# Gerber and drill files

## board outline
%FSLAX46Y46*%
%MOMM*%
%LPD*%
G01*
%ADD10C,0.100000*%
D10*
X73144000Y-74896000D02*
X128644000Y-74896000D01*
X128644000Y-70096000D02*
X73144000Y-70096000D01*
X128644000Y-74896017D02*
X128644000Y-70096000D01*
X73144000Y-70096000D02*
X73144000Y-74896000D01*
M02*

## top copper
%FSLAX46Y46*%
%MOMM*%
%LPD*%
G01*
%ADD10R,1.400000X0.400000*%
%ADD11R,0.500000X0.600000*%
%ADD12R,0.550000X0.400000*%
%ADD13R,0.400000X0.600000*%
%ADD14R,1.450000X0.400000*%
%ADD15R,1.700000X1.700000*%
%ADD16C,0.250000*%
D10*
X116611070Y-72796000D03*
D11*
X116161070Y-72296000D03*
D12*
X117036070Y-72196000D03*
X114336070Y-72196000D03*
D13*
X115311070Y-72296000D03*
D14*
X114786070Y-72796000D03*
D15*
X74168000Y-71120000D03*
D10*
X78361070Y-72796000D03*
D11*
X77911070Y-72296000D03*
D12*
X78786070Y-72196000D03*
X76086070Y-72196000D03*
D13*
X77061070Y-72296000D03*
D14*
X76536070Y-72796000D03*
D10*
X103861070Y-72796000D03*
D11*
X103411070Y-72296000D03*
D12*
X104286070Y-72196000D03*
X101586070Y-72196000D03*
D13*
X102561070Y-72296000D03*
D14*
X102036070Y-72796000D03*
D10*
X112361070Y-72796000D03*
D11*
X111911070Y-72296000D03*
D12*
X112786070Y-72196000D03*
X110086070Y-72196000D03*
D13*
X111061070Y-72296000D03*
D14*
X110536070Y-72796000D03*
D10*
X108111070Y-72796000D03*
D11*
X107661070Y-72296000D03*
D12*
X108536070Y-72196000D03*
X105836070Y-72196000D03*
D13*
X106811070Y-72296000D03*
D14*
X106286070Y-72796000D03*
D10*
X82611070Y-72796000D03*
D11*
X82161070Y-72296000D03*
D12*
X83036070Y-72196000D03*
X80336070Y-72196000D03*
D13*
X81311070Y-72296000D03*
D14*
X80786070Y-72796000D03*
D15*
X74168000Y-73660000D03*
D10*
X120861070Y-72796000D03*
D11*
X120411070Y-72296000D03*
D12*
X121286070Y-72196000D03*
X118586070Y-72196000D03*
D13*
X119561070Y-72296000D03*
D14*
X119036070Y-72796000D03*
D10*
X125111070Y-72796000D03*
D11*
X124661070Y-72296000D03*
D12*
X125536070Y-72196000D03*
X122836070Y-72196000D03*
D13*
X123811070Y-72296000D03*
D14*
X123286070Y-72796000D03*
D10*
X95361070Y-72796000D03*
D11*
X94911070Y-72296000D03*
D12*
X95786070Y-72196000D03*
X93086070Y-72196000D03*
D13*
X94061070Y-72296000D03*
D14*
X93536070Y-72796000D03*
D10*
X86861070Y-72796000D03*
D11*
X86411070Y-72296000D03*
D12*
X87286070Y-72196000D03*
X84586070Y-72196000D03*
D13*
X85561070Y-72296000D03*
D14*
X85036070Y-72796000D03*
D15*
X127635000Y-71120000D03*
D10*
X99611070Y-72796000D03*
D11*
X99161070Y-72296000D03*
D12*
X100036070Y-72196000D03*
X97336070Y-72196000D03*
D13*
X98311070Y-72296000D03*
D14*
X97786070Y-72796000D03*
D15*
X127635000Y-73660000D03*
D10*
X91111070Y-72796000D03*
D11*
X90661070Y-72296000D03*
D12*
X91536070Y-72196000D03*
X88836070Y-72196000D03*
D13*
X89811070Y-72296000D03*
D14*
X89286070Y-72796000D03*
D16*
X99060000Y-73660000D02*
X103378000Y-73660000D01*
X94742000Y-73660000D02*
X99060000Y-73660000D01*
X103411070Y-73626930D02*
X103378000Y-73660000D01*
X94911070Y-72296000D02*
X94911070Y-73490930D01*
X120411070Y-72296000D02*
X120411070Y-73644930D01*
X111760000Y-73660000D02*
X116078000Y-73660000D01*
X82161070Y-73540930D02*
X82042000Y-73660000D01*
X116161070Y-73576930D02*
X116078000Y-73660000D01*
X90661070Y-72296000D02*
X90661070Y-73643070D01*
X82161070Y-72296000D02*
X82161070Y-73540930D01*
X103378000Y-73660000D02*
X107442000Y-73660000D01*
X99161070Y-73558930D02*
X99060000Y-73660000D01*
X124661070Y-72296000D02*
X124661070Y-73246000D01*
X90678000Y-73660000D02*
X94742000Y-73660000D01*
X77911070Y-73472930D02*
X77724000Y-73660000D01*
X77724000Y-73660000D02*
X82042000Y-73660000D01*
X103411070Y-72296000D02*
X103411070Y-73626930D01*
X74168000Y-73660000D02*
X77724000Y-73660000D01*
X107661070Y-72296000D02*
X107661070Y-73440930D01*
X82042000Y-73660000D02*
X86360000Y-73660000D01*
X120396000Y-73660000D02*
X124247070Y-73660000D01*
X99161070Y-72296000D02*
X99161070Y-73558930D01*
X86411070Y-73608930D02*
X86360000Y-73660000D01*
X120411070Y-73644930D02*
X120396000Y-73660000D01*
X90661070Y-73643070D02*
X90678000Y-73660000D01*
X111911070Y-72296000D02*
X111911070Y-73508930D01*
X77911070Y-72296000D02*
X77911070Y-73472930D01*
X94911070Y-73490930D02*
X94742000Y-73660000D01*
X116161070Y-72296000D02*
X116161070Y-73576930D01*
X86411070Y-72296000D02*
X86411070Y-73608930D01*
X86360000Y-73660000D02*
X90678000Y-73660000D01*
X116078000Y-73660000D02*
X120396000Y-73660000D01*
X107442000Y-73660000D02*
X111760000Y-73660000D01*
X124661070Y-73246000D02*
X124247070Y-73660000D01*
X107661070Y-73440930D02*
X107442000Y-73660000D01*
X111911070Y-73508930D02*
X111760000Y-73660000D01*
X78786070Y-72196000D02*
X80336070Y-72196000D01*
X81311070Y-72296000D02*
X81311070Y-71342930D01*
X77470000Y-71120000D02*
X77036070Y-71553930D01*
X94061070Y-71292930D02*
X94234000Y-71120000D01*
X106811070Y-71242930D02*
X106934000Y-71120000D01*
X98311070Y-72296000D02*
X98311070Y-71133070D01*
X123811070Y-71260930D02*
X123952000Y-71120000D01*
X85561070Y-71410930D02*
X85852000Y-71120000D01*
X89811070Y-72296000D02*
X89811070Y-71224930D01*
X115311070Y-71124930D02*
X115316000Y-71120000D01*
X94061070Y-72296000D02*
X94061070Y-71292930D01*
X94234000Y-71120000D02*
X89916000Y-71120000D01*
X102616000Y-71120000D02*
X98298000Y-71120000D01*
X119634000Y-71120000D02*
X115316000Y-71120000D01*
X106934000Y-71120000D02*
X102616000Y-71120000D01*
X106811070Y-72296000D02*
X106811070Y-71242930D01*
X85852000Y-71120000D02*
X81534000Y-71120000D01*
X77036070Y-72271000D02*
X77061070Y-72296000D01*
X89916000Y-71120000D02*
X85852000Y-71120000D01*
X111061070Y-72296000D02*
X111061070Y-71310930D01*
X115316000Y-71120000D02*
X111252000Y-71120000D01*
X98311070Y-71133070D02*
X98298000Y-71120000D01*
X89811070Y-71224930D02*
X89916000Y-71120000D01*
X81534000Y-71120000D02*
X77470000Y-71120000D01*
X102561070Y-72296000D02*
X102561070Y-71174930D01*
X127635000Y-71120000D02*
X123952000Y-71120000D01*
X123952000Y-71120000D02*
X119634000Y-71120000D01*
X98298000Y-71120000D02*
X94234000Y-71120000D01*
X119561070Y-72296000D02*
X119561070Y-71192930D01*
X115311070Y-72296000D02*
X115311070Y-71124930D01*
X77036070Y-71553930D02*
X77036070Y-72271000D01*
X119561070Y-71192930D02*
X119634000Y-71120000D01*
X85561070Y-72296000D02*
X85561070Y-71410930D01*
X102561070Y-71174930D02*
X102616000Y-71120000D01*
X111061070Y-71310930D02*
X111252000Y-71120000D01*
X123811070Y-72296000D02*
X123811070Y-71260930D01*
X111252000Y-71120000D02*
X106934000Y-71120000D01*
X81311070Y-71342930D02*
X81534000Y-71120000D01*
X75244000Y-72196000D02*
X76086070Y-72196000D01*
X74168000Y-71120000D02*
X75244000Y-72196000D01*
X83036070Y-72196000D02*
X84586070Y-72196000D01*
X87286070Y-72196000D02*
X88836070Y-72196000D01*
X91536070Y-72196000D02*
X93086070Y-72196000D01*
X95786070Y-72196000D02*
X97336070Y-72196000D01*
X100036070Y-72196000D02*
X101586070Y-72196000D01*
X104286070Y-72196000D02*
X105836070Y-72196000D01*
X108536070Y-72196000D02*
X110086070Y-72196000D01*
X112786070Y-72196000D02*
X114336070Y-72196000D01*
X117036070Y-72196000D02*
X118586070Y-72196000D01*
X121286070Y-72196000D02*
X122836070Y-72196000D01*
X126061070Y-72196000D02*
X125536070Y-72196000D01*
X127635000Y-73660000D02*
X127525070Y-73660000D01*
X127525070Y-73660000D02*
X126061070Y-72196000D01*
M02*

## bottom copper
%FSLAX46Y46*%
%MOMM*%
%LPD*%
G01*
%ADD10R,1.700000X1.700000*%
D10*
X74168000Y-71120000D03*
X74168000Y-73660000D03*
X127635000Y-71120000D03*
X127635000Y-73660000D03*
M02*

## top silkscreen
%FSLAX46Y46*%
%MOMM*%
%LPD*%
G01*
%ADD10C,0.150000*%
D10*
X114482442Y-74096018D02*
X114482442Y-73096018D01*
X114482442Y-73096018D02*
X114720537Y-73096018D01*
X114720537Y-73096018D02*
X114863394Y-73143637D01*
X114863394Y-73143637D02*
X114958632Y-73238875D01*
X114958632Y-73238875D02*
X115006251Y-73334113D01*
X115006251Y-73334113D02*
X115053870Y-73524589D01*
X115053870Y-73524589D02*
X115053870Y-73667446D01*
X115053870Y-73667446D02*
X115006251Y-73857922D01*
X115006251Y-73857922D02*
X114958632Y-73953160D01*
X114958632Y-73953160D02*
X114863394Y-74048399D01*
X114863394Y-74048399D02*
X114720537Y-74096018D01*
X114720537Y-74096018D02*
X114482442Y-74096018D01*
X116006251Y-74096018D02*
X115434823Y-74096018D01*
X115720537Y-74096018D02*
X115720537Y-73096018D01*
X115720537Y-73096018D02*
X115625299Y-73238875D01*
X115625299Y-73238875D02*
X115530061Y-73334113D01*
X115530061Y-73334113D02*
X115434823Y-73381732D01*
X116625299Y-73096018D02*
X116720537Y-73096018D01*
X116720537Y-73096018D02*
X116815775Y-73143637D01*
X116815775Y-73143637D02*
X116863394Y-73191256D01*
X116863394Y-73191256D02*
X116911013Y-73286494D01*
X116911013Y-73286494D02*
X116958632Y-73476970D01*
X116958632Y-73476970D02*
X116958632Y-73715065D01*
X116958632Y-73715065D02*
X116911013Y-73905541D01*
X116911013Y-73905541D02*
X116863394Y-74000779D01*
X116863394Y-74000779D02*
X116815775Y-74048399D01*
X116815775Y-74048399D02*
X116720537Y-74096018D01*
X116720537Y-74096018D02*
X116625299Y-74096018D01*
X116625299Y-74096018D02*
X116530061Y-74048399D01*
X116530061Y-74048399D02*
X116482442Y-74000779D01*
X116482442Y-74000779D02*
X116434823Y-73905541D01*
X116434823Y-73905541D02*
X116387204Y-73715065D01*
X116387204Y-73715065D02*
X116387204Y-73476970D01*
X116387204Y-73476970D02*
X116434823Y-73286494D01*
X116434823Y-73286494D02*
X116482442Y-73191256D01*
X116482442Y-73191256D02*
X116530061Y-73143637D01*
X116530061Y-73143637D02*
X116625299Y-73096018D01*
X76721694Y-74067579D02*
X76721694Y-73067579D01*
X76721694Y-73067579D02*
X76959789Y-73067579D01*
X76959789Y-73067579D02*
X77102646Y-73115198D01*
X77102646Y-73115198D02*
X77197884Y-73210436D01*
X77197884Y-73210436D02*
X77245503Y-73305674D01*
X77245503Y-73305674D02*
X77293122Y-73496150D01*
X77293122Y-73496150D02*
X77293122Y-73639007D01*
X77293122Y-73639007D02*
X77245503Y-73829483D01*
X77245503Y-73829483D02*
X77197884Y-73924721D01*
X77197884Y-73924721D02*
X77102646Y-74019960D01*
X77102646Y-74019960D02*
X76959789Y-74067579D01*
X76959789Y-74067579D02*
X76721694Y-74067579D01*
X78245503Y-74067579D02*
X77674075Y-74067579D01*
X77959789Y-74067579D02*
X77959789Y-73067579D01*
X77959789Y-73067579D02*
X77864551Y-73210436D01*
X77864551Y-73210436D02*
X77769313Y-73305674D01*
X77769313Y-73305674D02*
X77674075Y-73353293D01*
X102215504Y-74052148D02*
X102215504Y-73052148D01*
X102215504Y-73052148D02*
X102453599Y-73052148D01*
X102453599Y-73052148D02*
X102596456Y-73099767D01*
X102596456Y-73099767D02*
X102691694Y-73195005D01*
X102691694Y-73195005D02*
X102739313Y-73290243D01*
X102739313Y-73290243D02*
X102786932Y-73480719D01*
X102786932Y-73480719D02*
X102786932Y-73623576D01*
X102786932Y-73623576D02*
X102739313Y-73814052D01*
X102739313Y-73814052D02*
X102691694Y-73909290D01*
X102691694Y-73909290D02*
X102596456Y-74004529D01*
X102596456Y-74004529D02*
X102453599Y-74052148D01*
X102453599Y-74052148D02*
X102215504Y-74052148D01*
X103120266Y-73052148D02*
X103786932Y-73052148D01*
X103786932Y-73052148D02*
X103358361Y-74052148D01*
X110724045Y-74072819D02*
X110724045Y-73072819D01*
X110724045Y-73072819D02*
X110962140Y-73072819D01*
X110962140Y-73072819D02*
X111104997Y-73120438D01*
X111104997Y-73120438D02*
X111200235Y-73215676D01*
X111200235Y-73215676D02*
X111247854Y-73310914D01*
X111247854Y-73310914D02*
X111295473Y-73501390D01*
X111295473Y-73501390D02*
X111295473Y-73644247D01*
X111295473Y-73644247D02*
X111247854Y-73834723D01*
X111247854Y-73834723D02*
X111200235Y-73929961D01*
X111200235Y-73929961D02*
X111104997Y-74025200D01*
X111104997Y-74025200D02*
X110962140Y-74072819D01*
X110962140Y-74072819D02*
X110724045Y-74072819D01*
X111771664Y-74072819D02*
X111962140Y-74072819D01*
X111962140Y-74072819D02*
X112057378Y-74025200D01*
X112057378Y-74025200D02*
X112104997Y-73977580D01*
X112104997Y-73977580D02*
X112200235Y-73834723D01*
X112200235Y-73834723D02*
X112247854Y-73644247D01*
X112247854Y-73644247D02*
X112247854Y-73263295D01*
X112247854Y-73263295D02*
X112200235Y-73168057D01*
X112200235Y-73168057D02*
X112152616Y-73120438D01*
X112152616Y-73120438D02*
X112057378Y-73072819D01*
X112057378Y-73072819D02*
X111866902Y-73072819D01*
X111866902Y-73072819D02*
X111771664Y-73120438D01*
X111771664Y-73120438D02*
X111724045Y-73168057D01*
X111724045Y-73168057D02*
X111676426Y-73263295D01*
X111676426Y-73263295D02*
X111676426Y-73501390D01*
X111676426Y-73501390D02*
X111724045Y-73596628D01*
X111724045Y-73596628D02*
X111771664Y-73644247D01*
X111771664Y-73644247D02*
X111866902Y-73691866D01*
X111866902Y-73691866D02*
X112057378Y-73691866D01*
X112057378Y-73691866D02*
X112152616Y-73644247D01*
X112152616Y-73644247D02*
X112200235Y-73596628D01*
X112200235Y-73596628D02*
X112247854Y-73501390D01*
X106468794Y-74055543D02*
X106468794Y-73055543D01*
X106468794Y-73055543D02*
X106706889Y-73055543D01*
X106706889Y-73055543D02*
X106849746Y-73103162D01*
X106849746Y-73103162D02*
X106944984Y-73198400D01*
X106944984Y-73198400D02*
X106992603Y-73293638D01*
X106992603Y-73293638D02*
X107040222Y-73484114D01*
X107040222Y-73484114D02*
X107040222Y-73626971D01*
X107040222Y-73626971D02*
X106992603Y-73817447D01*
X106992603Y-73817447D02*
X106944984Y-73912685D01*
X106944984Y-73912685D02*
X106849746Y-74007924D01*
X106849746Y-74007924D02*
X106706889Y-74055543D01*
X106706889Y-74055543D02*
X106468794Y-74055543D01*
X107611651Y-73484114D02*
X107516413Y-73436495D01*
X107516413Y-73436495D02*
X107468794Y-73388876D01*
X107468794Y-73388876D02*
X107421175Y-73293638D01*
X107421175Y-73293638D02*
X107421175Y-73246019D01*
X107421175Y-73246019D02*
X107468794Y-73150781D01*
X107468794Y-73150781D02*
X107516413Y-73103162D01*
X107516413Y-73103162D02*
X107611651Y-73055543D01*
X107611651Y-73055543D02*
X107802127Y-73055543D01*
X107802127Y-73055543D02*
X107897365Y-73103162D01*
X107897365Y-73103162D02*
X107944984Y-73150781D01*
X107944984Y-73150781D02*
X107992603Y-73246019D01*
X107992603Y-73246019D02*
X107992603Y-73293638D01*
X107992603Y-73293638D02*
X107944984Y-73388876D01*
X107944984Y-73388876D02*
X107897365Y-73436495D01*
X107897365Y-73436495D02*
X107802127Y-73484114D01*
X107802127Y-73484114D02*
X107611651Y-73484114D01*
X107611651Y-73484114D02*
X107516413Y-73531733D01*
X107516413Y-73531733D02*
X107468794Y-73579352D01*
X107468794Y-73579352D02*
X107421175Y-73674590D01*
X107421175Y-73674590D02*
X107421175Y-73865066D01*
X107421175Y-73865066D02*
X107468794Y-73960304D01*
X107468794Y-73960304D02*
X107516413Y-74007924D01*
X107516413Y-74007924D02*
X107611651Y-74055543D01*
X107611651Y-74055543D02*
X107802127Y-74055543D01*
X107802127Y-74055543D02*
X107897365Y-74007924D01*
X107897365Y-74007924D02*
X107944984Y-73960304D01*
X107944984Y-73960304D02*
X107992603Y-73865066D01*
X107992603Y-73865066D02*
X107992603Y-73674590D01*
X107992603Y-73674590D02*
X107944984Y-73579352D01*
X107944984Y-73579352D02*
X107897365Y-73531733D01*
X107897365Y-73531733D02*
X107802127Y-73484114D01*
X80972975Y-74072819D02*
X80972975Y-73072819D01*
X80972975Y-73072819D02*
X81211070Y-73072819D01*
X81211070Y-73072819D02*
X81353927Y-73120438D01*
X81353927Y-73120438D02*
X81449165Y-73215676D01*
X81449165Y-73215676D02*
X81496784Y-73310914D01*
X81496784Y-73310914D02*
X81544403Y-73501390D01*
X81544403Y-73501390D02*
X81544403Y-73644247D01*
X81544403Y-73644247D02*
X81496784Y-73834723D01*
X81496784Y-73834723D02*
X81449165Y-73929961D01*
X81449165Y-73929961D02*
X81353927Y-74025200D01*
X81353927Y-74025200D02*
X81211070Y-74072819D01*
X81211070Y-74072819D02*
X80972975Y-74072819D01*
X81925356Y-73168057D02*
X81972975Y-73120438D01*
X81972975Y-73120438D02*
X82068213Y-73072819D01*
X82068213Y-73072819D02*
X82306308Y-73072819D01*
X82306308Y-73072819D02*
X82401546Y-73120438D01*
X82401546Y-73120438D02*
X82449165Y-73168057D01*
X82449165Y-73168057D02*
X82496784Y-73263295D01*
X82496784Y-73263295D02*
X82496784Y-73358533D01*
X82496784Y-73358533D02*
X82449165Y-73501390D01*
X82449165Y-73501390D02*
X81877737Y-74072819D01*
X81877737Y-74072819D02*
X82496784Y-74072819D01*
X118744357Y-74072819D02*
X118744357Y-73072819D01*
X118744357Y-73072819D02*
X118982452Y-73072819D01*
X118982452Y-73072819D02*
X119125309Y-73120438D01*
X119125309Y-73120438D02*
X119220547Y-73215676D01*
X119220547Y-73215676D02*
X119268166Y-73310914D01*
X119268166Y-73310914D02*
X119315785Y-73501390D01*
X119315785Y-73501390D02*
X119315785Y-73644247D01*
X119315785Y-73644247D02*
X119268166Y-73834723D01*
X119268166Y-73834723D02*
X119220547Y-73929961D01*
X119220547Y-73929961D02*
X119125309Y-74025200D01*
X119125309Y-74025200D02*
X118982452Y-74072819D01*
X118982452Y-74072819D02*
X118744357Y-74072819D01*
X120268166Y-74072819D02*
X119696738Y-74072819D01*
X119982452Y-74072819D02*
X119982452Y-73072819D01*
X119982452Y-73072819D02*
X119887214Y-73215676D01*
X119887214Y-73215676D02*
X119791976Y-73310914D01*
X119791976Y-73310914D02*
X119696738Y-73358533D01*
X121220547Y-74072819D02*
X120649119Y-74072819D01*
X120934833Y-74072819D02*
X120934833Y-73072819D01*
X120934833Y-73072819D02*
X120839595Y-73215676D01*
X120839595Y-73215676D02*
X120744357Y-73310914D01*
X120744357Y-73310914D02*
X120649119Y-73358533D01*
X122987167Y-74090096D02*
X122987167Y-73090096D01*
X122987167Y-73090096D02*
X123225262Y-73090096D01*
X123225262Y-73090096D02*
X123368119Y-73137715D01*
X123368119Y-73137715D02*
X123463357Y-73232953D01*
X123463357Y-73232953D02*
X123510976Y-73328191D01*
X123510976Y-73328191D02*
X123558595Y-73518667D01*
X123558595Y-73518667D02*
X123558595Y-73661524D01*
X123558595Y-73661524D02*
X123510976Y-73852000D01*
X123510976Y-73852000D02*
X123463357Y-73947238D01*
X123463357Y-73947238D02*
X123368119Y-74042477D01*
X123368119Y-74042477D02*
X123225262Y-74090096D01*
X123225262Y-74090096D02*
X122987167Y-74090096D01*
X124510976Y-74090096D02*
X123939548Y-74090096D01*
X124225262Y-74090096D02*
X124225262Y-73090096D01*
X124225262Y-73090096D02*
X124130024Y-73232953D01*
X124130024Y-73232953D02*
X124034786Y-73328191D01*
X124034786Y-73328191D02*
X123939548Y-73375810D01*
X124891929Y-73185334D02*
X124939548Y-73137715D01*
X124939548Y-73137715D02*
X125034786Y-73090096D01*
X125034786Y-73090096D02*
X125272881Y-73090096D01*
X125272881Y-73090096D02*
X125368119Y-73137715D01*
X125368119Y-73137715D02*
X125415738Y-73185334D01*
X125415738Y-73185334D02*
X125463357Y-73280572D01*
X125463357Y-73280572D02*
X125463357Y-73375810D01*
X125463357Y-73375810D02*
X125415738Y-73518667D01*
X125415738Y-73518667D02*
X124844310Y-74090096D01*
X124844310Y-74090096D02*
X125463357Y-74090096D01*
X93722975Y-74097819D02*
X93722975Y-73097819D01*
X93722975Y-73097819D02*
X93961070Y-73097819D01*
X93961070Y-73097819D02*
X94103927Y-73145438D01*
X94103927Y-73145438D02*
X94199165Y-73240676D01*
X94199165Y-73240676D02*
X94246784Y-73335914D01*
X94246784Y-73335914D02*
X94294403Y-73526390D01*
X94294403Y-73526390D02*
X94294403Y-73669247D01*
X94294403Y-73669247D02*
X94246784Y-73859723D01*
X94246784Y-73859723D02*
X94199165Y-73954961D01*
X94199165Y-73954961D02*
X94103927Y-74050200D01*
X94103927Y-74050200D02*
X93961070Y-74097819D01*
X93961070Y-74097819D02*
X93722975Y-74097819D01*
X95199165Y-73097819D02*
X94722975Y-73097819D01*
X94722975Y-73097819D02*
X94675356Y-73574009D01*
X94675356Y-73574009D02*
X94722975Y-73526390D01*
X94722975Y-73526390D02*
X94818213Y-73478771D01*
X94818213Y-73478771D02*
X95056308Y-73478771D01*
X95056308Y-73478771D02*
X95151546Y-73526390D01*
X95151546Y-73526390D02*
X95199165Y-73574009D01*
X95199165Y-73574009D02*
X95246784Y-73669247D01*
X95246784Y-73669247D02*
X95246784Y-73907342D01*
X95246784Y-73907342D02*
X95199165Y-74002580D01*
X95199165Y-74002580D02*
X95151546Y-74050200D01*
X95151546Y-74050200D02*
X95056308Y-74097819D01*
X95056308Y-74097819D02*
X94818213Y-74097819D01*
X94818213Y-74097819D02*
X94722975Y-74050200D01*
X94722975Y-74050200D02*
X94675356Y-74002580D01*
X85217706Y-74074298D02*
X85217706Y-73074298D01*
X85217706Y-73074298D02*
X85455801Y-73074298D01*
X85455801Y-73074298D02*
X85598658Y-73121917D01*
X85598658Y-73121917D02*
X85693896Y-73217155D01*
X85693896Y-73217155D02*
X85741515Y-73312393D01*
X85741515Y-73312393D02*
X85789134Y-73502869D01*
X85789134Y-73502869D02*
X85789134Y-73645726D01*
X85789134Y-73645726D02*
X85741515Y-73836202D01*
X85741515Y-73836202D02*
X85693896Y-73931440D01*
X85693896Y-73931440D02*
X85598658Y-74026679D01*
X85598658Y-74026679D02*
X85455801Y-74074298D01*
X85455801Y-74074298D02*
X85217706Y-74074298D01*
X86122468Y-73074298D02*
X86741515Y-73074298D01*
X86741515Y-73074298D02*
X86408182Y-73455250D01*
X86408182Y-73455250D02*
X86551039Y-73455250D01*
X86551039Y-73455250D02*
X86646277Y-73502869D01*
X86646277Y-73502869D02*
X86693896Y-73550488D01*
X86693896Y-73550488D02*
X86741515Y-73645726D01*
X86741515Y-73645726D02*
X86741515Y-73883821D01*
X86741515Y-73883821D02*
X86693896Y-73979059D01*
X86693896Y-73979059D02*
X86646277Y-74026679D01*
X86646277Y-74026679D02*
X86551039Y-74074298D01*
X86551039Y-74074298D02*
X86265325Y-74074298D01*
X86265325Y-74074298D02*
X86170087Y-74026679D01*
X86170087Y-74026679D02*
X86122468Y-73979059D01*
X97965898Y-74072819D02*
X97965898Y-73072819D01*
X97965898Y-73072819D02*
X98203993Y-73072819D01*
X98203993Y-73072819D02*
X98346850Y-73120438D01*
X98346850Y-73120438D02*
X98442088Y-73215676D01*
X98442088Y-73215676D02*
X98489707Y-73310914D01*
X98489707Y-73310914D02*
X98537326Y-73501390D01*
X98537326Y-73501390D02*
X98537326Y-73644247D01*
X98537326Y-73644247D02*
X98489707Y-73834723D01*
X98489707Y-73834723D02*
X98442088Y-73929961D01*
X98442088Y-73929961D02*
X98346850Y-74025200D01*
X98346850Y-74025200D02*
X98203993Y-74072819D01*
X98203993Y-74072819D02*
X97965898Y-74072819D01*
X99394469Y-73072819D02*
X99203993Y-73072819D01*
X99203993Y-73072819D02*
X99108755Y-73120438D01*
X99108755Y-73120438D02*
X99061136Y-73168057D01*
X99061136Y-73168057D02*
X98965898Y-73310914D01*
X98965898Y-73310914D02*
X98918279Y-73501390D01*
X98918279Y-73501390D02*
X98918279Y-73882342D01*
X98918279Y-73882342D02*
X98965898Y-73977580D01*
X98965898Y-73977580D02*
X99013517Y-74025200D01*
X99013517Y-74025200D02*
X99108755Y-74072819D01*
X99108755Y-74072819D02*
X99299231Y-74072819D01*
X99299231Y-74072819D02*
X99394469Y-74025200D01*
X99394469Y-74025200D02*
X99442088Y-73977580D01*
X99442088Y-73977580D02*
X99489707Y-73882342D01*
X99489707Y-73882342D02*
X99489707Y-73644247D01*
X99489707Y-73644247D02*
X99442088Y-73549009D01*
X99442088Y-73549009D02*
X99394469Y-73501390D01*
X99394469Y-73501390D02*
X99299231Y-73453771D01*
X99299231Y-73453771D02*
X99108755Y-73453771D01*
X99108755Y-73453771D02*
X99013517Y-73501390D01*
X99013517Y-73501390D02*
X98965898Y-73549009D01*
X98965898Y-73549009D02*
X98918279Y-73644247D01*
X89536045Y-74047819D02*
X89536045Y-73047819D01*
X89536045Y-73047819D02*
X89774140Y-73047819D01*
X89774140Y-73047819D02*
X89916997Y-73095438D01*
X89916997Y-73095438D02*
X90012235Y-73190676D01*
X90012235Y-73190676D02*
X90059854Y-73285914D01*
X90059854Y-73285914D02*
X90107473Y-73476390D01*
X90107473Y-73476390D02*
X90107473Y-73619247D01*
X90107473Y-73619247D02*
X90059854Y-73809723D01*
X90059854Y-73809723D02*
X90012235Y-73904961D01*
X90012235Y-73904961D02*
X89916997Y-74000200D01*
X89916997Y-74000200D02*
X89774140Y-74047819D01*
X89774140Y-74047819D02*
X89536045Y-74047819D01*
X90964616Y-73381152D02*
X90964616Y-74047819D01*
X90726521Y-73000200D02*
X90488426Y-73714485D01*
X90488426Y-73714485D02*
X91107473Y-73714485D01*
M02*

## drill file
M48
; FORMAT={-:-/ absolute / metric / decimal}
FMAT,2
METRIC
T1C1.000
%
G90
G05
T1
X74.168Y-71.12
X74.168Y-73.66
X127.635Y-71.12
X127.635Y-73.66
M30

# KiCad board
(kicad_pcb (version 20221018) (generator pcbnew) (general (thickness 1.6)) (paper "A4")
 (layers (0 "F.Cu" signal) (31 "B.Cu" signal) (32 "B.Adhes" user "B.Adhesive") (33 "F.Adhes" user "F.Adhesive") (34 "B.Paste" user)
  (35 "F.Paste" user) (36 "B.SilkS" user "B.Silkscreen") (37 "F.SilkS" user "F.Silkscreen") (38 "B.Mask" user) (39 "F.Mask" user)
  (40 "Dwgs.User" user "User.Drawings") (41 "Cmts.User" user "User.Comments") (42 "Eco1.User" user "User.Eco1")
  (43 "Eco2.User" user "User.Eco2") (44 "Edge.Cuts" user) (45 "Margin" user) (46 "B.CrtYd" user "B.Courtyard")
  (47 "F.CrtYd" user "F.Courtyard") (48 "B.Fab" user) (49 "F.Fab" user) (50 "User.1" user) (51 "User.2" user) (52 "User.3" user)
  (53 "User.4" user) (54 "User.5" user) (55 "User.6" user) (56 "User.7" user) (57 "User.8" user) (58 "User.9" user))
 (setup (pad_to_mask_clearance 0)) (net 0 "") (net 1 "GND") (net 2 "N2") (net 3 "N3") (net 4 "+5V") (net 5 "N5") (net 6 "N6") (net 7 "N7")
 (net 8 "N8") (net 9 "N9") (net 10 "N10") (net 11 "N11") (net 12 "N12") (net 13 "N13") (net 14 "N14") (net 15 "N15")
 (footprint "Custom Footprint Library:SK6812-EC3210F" (layer "F.Cu") (at 115.71107 72.496 180)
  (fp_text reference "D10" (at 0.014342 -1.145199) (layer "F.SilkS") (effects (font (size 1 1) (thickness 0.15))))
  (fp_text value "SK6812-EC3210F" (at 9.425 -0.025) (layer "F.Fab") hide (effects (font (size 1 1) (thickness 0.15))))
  (pad "1" smd rect (at -0.9 -0.3) (size 1.4 0.4) (layers "F.Cu" "F.Paste" "F.Mask") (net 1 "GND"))
  (pad "1" smd rect (at -0.45 0.2) (size 0.5 0.6) (layers "F.Cu" "F.Paste" "F.Mask") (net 1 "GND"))
  (pad "2" smd rect (at -1.325 0.3) (size 0.55 0.4) (layers "F.Cu" "F.Paste" "F.Mask") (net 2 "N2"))
  (pad "3" smd rect (at 1.375 0.3) (size 0.55 0.4) (layers "F.Cu" "F.Paste" "F.Mask") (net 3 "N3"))
  (pad "4" smd rect (at 0.4 0.2) (size 0.4 0.6) (layers "F.Cu" "F.Paste" "F.Mask") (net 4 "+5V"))
  (pad "4" smd rect (at 0.925 -0.3) (size 1.45 0.4) (layers "F.Cu" "F.Paste" "F.Mask") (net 4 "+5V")))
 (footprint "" (layer "F.Cu") (at 74.168 71.12)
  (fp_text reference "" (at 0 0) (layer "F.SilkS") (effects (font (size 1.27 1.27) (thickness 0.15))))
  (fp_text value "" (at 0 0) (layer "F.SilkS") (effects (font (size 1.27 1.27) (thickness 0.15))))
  (pad "1" thru_hole rect (at 0 0) (size 1.7 1.7) (drill 1) (layers "*.Cu" "*.Mask") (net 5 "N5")))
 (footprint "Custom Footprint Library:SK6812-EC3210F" (layer "F.Cu") (at 77.46107 72.496 180)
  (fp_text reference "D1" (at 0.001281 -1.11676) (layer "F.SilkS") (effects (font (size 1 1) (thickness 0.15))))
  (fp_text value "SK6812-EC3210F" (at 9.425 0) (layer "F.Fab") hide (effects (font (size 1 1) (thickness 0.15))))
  (pad "1" smd rect (at -0.9 -0.3) (size 1.4 0.4) (layers "F.Cu" "F.Paste" "F.Mask") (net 1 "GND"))
  (pad "1" smd rect (at -0.45 0.2) (size 0.5 0.6) (layers "F.Cu" "F.Paste" "F.Mask") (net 1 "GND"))
  (pad "2" smd rect (at -1.325 0.3) (size 0.55 0.4) (layers "F.Cu" "F.Paste" "F.Mask") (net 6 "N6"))
  (pad "3" smd rect (at 1.375 0.3) (size 0.55 0.4) (layers "F.Cu" "F.Paste" "F.Mask") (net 5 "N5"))
  (pad "4" smd rect (at 0.4 0.2) (size 0.4 0.6) (layers "F.Cu" "F.Paste" "F.Mask") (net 4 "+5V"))
  (pad "4" smd rect (at 0.925 -0.3) (size 1.45 0.4) (layers "F.Cu" "F.Paste" "F.Mask") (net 4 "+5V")))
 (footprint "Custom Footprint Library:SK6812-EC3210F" (layer "F.Cu") (at 102.96107 72.496 180)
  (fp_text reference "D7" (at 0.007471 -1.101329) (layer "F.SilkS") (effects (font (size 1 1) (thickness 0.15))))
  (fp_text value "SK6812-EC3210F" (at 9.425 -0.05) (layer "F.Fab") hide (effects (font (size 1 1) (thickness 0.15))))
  (pad "1" smd rect (at -0.9 -0.3) (size 1.4 0.4) (layers "F.Cu" "F.Paste" "F.Mask") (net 1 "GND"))
  (pad "1" smd rect (at -0.45 0.2) (size 0.5 0.6) (layers "F.Cu" "F.Paste" "F.Mask") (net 1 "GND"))
  (pad "2" smd rect (at -1.325 0.3) (size 0.55 0.4) (layers "F.Cu" "F.Paste" "F.Mask") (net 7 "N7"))
  (pad "3" smd rect (at 1.375 0.3) (size 0.55 0.4) (layers "F.Cu" "F.Paste" "F.Mask") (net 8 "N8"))
  (pad "4" smd rect (at 0.4 0.2) (size 0.4 0.6) (layers "F.Cu" "F.Paste" "F.Mask") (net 4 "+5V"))
  (pad "4" smd rect (at 0.925 -0.3) (size 1.45 0.4) (layers "F.Cu" "F.Paste" "F.Mask") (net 4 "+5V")))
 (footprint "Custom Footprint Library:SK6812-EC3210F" (layer "F.Cu") (at 111.46107 72.496 180)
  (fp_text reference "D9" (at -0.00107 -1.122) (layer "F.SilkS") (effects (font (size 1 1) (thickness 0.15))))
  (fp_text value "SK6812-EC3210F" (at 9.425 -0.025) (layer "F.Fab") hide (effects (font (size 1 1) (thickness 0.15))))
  (pad "1" smd rect (at -0.9 -0.3) (size 1.4 0.4) (layers "F.Cu" "F.Paste" "F.Mask") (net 1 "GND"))
  (pad "1" smd rect (at -0.45 0.2) (size 0.5 0.6) (layers "F.Cu" "F.Paste" "F.Mask") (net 1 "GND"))
  (pad "2" smd rect (at -1.325 0.3) (size 0.55 0.4) (layers "F.Cu" "F.Paste" "F.Mask") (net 3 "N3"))
  (pad "3" smd rect (at 1.375 0.3) (size 0.55 0.4) (layers "F.Cu" "F.Paste" "F.Mask") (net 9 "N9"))
  (pad "4" smd rect (at 0.4 0.2) (size 0.4 0.6) (layers "F.Cu" "F.Paste" "F.Mask") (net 4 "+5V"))
  (pad "4" smd rect (at 0.925 -0.3) (size 1.45 0.4) (layers "F.Cu" "F.Paste" "F.Mask") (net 4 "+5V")))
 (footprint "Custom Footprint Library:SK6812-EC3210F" (layer "F.Cu") (at 107.21107 72.496 180)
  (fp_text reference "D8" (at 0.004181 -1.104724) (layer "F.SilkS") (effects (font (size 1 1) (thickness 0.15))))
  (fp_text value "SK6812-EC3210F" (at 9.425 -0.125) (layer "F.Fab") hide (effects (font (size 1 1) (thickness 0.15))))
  (pad "1" smd rect (at -0.9 -0.3) (size 1.4 0.4) (layers "F.Cu" "F.Paste" "F.Mask") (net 1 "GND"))
  (pad "1" smd rect (at -0.45 0.2) (size 0.5 0.6) (layers "F.Cu" "F.Paste" "F.Mask") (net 1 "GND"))
  (pad "2" smd rect (at -1.325 0.3) (size 0.55 0.4) (layers "F.Cu" "F.Paste" "F.Mask") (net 9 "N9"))
  (pad "3" smd rect (at 1.375 0.3) (size 0.55 0.4) (layers "F.Cu" "F.Paste" "F.Mask") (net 7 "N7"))
  (pad "4" smd rect (at 0.4 0.2) (size 0.4 0.6) (layers "F.Cu" "F.Paste" "F.Mask") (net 4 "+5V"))
  (pad "4" smd rect (at 0.925 -0.3) (size 1.45 0.4) (layers "F.Cu" "F.Paste" "F.Mask") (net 4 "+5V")))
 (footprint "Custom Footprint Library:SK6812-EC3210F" (layer "F.Cu") (at 81.71107 72.496 180)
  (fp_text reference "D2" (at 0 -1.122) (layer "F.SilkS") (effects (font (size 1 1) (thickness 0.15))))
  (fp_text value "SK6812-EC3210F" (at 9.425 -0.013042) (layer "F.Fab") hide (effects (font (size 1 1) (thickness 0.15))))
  (pad "1" smd rect (at -0.9 -0.3) (size 1.4 0.4) (layers "F.Cu" "F.Paste" "F.Mask") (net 1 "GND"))
  (pad "1" smd rect (at -0.45 0.2) (size 0.5 0.6) (layers "F.Cu" "F.Paste" "F.Mask") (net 1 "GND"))
  (pad "2" smd rect (at -1.325 0.3) (size 0.55 0.4) (layers "F.Cu" "F.Paste" "F.Mask") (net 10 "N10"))
  (pad "3" smd rect (at 1.375 0.3) (size 0.55 0.4) (layers "F.Cu" "F.Paste" "F.Mask") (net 6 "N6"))
  (pad "4" smd rect (at 0.4 0.2) (size 0.4 0.6) (layers "F.Cu" "F.Paste" "F.Mask") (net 4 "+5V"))
  (pad "4" smd rect (at 0.925 -0.3) (size 1.45 0.4) (layers "F.Cu" "F.Paste" "F.Mask") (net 4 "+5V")))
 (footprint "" (layer "F.Cu") (at 74.168 73.66)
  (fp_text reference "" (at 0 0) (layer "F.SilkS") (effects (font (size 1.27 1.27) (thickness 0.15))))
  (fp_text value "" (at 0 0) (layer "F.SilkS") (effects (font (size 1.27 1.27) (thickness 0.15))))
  (pad "1" thru_hole rect (at 0 0) (size 1.7 1.7) (drill 1) (layers "*.Cu" "*.Mask") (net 1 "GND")))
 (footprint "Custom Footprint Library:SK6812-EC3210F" (layer "F.Cu") (at 119.96107 72.496 180)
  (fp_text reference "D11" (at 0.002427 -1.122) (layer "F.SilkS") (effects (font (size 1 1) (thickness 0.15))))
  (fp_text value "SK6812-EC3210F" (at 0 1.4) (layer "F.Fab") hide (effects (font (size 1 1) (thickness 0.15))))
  (pad "1" smd rect (at -0.9 -0.3) (size 1.4 0.4) (layers "F.Cu" "F.Paste" "F.Mask") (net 1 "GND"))
  (pad "1" smd rect (at -0.45 0.2) (size 0.5 0.6) (layers "F.Cu" "F.Paste" "F.Mask") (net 1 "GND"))
  (pad "2" smd rect (at -1.325 0.3) (size 0.55 0.4) (layers "F.Cu" "F.Paste" "F.Mask") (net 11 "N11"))
  (pad "3" smd rect (at 1.375 0.3) (size 0.55 0.4) (layers "F.Cu" "F.Paste" "F.Mask") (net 2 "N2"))
  (pad "4" smd rect (at 0.4 0.2) (size 0.4 0.6) (layers "F.Cu" "F.Paste" "F.Mask") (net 4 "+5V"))
  (pad "4" smd rect (at 0.925 -0.3) (size 1.45 0.4) (layers "F.Cu" "F.Paste" "F.Mask") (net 4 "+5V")))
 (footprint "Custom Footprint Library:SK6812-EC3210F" (layer "F.Cu") (at 124.21107 72.496 180)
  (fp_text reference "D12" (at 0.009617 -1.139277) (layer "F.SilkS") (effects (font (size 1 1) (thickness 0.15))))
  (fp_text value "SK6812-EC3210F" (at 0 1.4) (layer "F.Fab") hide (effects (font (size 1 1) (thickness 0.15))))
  (pad "1" smd rect (at -0.9 -0.3) (size 1.4 0.4) (layers "F.Cu" "F.Paste" "F.Mask") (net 1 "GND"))
  (pad "1" smd rect (at -0.45 0.2) (size 0.5 0.6) (layers "F.Cu" "F.Paste" "F.Mask") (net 1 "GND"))
  (pad "2" smd rect (at -1.325 0.3) (size 0.55 0.4) (layers "F.Cu" "F.Paste" "F.Mask") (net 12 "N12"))
  (pad "3" smd rect (at 1.375 0.3) (size 0.55 0.4) (layers "F.Cu" "F.Paste" "F.Mask") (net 11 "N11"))
  (pad "4" smd rect (at 0.4 0.2) (size 0.4 0.6) (layers "F.Cu" "F.Paste" "F.Mask") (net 4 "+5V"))
  (pad "4" smd rect (at 0.925 -0.3) (size 1.45 0.4) (layers "F.Cu" "F.Paste" "F.Mask") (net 4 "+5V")))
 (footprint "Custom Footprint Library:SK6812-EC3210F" (layer "F.Cu") (at 94.46107 72.496 180)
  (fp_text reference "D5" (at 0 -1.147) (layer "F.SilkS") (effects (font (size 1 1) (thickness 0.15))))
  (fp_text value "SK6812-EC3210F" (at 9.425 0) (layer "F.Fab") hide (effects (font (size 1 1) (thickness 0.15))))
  (pad "1" smd rect (at -0.9 -0.3) (size 1.4 0.4) (layers "F.Cu" "F.Paste" "F.Mask") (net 1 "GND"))
  (pad "1" smd rect (at -0.45 0.2) (size 0.5 0.6) (layers "F.Cu" "F.Paste" "F.Mask") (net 1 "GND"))
  (pad "2" smd rect (at -1.325 0.3) (size 0.55 0.4) (layers "F.Cu" "F.Paste" "F.Mask") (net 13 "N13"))
  (pad "3" smd rect (at 1.375 0.3) (size 0.55 0.4) (layers "F.Cu" "F.Paste" "F.Mask") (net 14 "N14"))
  (pad "4" smd rect (at 0.4 0.2) (size 0.4 0.6) (layers "F.Cu" "F.Paste" "F.Mask") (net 4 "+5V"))
  (pad "4" smd rect (at 0.925 -0.3) (size 1.45 0.4) (layers "F.Cu" "F.Paste" "F.Mask") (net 4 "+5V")))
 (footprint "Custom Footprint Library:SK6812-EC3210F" (layer "F.Cu") (at 85.96107 72.496 180)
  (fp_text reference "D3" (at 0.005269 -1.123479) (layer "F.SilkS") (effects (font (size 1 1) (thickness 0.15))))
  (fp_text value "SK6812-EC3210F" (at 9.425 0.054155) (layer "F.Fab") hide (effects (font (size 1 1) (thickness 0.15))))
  (pad "1" smd rect (at -0.9 -0.3) (size 1.4 0.4) (layers "F.Cu" "F.Paste" "F.Mask") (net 1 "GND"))
  (pad "1" smd rect (at -0.45 0.2) (size 0.5 0.6) (layers "F.Cu" "F.Paste" "F.Mask") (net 1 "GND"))
  (pad "2" smd rect (at -1.325 0.3) (size 0.55 0.4) (layers "F.Cu" "F.Paste" "F.Mask") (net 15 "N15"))
  (pad "3" smd rect (at 1.375 0.3) (size 0.55 0.4) (layers "F.Cu" "F.Paste" "F.Mask") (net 10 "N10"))
  (pad "4" smd rect (at 0.4 0.2) (size 0.4 0.6) (layers "F.Cu" "F.Paste" "F.Mask") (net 4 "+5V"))
  (pad "4" smd rect (at 0.925 -0.3) (size 1.45 0.4) (layers "F.Cu" "F.Paste" "F.Mask") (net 4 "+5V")))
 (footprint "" (layer "F.Cu") (at 127.635 71.12)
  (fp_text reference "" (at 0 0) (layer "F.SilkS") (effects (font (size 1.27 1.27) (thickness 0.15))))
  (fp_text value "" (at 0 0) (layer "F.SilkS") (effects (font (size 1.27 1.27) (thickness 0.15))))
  (pad "1" thru_hole rect (at 0 0) (size 1.7 1.7) (drill 1) (layers "*.Cu" "*.Mask") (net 4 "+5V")))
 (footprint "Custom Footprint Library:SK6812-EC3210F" (layer "F.Cu") (at 98.71107 72.496 180)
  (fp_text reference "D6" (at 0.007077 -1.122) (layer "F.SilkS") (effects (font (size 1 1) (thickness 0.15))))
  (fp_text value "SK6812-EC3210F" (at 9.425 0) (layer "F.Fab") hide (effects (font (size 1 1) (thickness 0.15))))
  (pad "1" smd rect (at -0.9 -0.3) (size 1.4 0.4) (layers "F.Cu" "F.Paste" "F.Mask") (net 1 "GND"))
  (pad "1" smd rect (at -0.45 0.2) (size 0.5 0.6) (layers "F.Cu" "F.Paste" "F.Mask") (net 1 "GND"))
  (pad "2" smd rect (at -1.325 0.3) (size 0.55 0.4) (layers "F.Cu" "F.Paste" "F.Mask") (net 8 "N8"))
  (pad "3" smd rect (at 1.375 0.3) (size 0.55 0.4) (layers "F.Cu" "F.Paste" "F.Mask") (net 13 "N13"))
  (pad "4" smd rect (at 0.4 0.2) (size 0.4 0.6) (layers "F.Cu" "F.Paste" "F.Mask") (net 4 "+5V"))
  (pad "4" smd rect (at 0.925 -0.3) (size 1.45 0.4) (layers "F.Cu" "F.Paste" "F.Mask") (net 4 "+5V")))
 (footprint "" (layer "F.Cu") (at 127.635 73.66)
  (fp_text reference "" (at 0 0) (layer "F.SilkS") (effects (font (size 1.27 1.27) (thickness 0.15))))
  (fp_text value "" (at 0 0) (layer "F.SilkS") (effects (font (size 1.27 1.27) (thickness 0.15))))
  (pad "1" thru_hole rect (at 0 0) (size 1.7 1.7) (drill 1) (layers "*.Cu" "*.Mask") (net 12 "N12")))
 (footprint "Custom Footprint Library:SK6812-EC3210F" (layer "F.Cu") (at 90.21107 72.496 180)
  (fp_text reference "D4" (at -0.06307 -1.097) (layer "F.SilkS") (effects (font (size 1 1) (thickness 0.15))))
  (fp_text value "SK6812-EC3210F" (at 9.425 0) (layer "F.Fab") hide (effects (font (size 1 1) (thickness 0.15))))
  (pad "1" smd rect (at -0.9 -0.3) (size 1.4 0.4) (layers "F.Cu" "F.Paste" "F.Mask") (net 1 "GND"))
  (pad "1" smd rect (at -0.45 0.2) (size 0.5 0.6) (layers "F.Cu" "F.Paste" "F.Mask") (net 1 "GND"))
  (pad "2" smd rect (at -1.325 0.3) (size 0.55 0.4) (layers "F.Cu" "F.Paste" "F.Mask") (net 14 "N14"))
  (pad "3" smd rect (at 1.375 0.3) (size 0.55 0.4) (layers "F.Cu" "F.Paste" "F.Mask") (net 15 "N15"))
  (pad "4" smd rect (at 0.4 0.2) (size 0.4 0.6) (layers "F.Cu" "F.Paste" "F.Mask") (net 4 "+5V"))
  (pad "4" smd rect (at 0.925 -0.3) (size 1.45 0.4) (layers "F.Cu" "F.Paste" "F.Mask") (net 4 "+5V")))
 (gr_line (start 73.144 74.896) (end 128.644 74.896) (stroke (width 0.1) (type solid)) (layer "Edge.Cuts"))
 (gr_line (start 128.644 70.096) (end 73.144 70.096) (stroke (width 0.1) (type solid)) (layer "Edge.Cuts"))
 (gr_line (start 128.644 74.896017) (end 128.644 70.096) (stroke (width 0.1) (type solid)) (layer "Edge.Cuts"))
 (gr_line (start 73.144 70.096) (end 73.144 74.896) (stroke (width 0.1) (type solid)) (layer "Edge.Cuts"))
 (segment (start 99.06 73.66) (end 103.378 73.66) (width 0.25) (layer "F.Cu") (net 1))
 (segment (start 94.742 73.66) (end 99.06 73.66) (width 0.25) (layer "F.Cu") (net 1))
 (segment (start 103.41107 73.62693) (end 103.378 73.66) (width 0.25) (layer "F.Cu") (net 1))
 (segment (start 94.91107 72.296) (end 94.91107 73.49093) (width 0.25) (layer "F.Cu") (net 1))
 (segment (start 120.41107 72.296) (end 120.41107 73.64493) (width 0.25) (layer "F.Cu") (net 1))
 (segment (start 111.76 73.66) (end 116.078 73.66) (width 0.25) (layer "F.Cu") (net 1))
 (segment (start 82.16107 73.54093) (end 82.042 73.66) (width 0.25) (layer "F.Cu") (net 1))
 (segment (start 116.16107 73.57693) (end 116.078 73.66) (width 0.25) (layer "F.Cu") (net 1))
 (segment (start 90.66107 72.296) (end 90.66107 73.64307) (width 0.25) (layer "F.Cu") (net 1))
 (segment (start 82.16107 72.296) (end 82.16107 73.54093) (width 0.25) (layer "F.Cu") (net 1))
 (segment (start 103.378 73.66) (end 107.442 73.66) (width 0.25) (layer "F.Cu") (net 1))
 (segment (start 99.16107 73.55893) (end 99.06 73.66) (width 0.25) (layer "F.Cu") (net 1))
 (segment (start 124.66107 72.296) (end 124.66107 73.246) (width 0.25) (layer "F.Cu") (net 1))
 (segment (start 90.678 73.66) (end 94.742 73.66) (width 0.25) (layer "F.Cu") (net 1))
 (segment (start 77.91107 73.47293) (end 77.724 73.66) (width 0.25) (layer "F.Cu") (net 1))
 (segment (start 77.724 73.66) (end 82.042 73.66) (width 0.25) (layer "F.Cu") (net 1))
 (segment (start 103.41107 72.296) (end 103.41107 73.62693) (width 0.25) (layer "F.Cu") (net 1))
 (segment (start 74.168 73.66) (end 77.724 73.66) (width 0.25) (layer "F.Cu") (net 1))
 (segment (start 107.66107 72.296) (end 107.66107 73.44093) (width 0.25) (layer "F.Cu") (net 1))
 (segment (start 82.042 73.66) (end 86.36 73.66) (width 0.25) (layer "F.Cu") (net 1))
 (segment (start 120.396 73.66) (end 124.24707 73.66) (width 0.25) (layer "F.Cu") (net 1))
 (segment (start 99.16107 72.296) (end 99.16107 73.55893) (width 0.25) (layer "F.Cu") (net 1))
 (segment (start 86.41107 73.60893) (end 86.36 73.66) (width 0.25) (layer "F.Cu") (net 1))
 (segment (start 120.41107 73.64493) (end 120.396 73.66) (width 0.25) (layer "F.Cu") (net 1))
 (segment (start 90.66107 73.64307) (end 90.678 73.66) (width 0.25) (layer "F.Cu") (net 1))
 (segment (start 111.91107 72.296) (end 111.91107 73.50893) (width 0.25) (layer "F.Cu") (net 1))
 (segment (start 77.91107 72.296) (end 77.91107 73.47293) (width 0.25) (layer "F.Cu") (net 1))
 (segment (start 94.91107 73.49093) (end 94.742 73.66) (width 0.25) (layer "F.Cu") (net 1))
 (segment (start 116.16107 72.296) (end 116.16107 73.57693) (width 0.25) (layer "F.Cu") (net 1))
 (segment (start 86.41107 72.296) (end 86.41107 73.60893) (width 0.25) (layer "F.Cu") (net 1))
 (segment (start 86.36 73.66) (end 90.678 73.66) (width 0.25) (layer "F.Cu") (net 1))
 (segment (start 116.078 73.66) (end 120.396 73.66) (width 0.25) (layer "F.Cu") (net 1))
 (segment (start 107.442 73.66) (end 111.76 73.66) (width 0.25) (layer "F.Cu") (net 1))
 (segment (start 124.66107 73.246) (end 124.24707 73.66) (width 0.25) (layer "F.Cu") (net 1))
 (segment (start 107.66107 73.44093) (end 107.442 73.66) (width 0.25) (layer "F.Cu") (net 1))
 (segment (start 111.91107 73.50893) (end 111.76 73.66) (width 0.25) (layer "F.Cu") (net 1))
 (segment (start 78.78607 72.196) (end 80.33607 72.196) (width 0.25) (layer "F.Cu") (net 6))
 (segment (start 81.31107 72.296) (end 81.31107 71.34293) (width 0.25) (layer "F.Cu") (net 4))
 (segment (start 77.47 71.12) (end 77.03607 71.55393) (width 0.25) (layer "F.Cu") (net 4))
 (segment (start 94.06107 71.29293) (end 94.234 71.12) (width 0.25) (layer "F.Cu") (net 4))
 (segment (start 106.81107 71.24293) (end 106.934 71.12) (width 0.25) (layer "F.Cu") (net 4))
 (segment (start 98.31107 72.296) (end 98.31107 71.13307) (width 0.25) (layer "F.Cu") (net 4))
 (segment (start 123.81107 71.26093) (end 123.952 71.12) (width 0.25) (layer "F.Cu") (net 4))
 (segment (start 85.56107 71.41093) (end 85.852 71.12) (width 0.25) (layer "F.Cu") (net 4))
 (segment (start 89.81107 72.296) (end 89.81107 71.22493) (width 0.25) (layer "F.Cu") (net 4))
 (segment (start 115.31107 71.12493) (end 115.316 71.12) (width 0.25) (layer "F.Cu") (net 4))
 (segment (start 94.06107 72.296) (end 94.06107 71.29293) (width 0.25) (layer "F.Cu") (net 4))
 (segment (start 94.234 71.12) (end 89.916 71.12) (width 0.25) (layer "F.Cu") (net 4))
 (segment (start 102.616 71.12) (end 98.298 71.12) (width 0.25) (layer "F.Cu") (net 4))
 (segment (start 119.634 71.12) (end 115.316 71.12) (width 0.25) (layer "F.Cu") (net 4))
 (segment (start 106.934 71.12) (end 102.616 71.12) (width 0.25) (layer "F.Cu") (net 4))
 (segment (start 106.81107 72.296) (end 106.81107 71.24293) (width 0.25) (layer "F.Cu") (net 4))
 (segment (start 85.852 71.12) (end 81.534 71.12) (width 0.25) (layer "F.Cu") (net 4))
 (segment (start 77.03607 72.271) (end 77.06107 72.296) (width 0.25) (layer "F.Cu") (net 4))
 (segment (start 89.916 71.12) (end 85.852 71.12) (width 0.25) (layer "F.Cu") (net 4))
 (segment (start 111.06107 72.296) (end 111.06107 71.31093) (width 0.25) (layer "F.Cu") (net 4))
 (segment (start 115.316 71.12) (end 111.252 71.12) (width 0.25) (layer "F.Cu") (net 4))
 (segment (start 98.31107 71.13307) (end 98.298 71.12) (width 0.25) (layer "F.Cu") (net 4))
 (segment (start 89.81107 71.22493) (end 89.916 71.12) (width 0.25) (layer "F.Cu") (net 4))
 (segment (start 81.534 71.12) (end 77.47 71.12) (width 0.25) (layer "F.Cu") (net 4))
 (segment (start 102.56107 72.296) (end 102.56107 71.17493) (width 0.25) (layer "F.Cu") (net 4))
 (segment (start 127.635 71.12) (end 123.952 71.12) (width 0.25) (layer "F.Cu") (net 4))
 (segment (start 123.952 71.12) (end 119.634 71.12) (width 0.25) (layer "F.Cu") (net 4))
 (segment (start 98.298 71.12) (end 94.234 71.12) (width 0.25) (layer "F.Cu") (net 4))
 (segment (start 119.56107 72.296) (end 119.56107 71.19293) (width 0.25) (layer "F.Cu") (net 4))
 (segment (start 115.31107 72.296) (end 115.31107 71.12493) (width 0.25) (layer "F.Cu") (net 4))
 (segment (start 77.03607 71.55393) (end 77.03607 72.271) (width 0.25) (layer "F.Cu") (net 4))
 (segment (start 119.56107 71.19293) (end 119.634 71.12) (width 0.25) (layer "F.Cu") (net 4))
 (segment (start 85.56107 72.296) (end 85.56107 71.41093) (width 0.25) (layer "F.Cu") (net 4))
 (segment (start 102.56107 71.17493) (end 102.616 71.12) (width 0.25) (layer "F.Cu") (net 4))
 (segment (start 111.06107 71.31093) (end 111.252 71.12) (width 0.25) (layer "F.Cu") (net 4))
 (segment (start 123.81107 72.296) (end 123.81107 71.26093) (width 0.25) (layer "F.Cu") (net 4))
 (segment (start 111.252 71.12) (end 106.934 71.12) (width 0.25) (layer "F.Cu") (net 4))
 (segment (start 81.31107 71.34293) (end 81.534 71.12) (width 0.25) (layer "F.Cu") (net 4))
 (segment (start 75.244 72.196) (end 76.08607 72.196) (width 0.25) (layer "F.Cu") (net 5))
 (segment (start 74.168 71.12) (end 75.244 72.196) (width 0.25) (layer "F.Cu") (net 5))
 (segment (start 83.03607 72.196) (end 84.58607 72.196) (width 0.25) (layer "F.Cu") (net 10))
 (segment (start 87.28607 72.196) (end 88.83607 72.196) (width 0.25) (layer "F.Cu") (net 15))
 (segment (start 91.53607 72.196) (end 93.08607 72.196) (width 0.25) (layer "F.Cu") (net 14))
 (segment (start 95.78607 72.196) (end 97.33607 72.196) (width 0.25) (layer "F.Cu") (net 13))
 (segment (start 100.03607 72.196) (end 101.58607 72.196) (width 0.25) (layer "F.Cu") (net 8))
 (segment (start 104.28607 72.196) (end 105.83607 72.196) (width 0.25) (layer "F.Cu") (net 7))
 (segment (start 108.53607 72.196) (end 110.08607 72.196) (width 0.25) (layer "F.Cu") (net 9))
 (segment (start 112.78607 72.196) (end 114.33607 72.196) (width 0.25) (layer "F.Cu") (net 3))
 (segment (start 117.03607 72.196) (end 118.58607 72.196) (width 0.25) (layer "F.Cu") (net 2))
 (segment (start 121.28607 72.196) (end 122.83607 72.196) (width 0.25) (layer "F.Cu") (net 11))
 (segment (start 126.06107 72.196) (end 125.53607 72.196) (width 0.25) (layer "F.Cu") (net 12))
 (segment (start 127.635 73.66) (end 127.52507 73.66) (width 0.25) (layer "F.Cu") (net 12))
 (segment (start 127.52507 73.66) (end 126.06107 72.196) (width 0.25) (layer "F.Cu") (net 12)))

